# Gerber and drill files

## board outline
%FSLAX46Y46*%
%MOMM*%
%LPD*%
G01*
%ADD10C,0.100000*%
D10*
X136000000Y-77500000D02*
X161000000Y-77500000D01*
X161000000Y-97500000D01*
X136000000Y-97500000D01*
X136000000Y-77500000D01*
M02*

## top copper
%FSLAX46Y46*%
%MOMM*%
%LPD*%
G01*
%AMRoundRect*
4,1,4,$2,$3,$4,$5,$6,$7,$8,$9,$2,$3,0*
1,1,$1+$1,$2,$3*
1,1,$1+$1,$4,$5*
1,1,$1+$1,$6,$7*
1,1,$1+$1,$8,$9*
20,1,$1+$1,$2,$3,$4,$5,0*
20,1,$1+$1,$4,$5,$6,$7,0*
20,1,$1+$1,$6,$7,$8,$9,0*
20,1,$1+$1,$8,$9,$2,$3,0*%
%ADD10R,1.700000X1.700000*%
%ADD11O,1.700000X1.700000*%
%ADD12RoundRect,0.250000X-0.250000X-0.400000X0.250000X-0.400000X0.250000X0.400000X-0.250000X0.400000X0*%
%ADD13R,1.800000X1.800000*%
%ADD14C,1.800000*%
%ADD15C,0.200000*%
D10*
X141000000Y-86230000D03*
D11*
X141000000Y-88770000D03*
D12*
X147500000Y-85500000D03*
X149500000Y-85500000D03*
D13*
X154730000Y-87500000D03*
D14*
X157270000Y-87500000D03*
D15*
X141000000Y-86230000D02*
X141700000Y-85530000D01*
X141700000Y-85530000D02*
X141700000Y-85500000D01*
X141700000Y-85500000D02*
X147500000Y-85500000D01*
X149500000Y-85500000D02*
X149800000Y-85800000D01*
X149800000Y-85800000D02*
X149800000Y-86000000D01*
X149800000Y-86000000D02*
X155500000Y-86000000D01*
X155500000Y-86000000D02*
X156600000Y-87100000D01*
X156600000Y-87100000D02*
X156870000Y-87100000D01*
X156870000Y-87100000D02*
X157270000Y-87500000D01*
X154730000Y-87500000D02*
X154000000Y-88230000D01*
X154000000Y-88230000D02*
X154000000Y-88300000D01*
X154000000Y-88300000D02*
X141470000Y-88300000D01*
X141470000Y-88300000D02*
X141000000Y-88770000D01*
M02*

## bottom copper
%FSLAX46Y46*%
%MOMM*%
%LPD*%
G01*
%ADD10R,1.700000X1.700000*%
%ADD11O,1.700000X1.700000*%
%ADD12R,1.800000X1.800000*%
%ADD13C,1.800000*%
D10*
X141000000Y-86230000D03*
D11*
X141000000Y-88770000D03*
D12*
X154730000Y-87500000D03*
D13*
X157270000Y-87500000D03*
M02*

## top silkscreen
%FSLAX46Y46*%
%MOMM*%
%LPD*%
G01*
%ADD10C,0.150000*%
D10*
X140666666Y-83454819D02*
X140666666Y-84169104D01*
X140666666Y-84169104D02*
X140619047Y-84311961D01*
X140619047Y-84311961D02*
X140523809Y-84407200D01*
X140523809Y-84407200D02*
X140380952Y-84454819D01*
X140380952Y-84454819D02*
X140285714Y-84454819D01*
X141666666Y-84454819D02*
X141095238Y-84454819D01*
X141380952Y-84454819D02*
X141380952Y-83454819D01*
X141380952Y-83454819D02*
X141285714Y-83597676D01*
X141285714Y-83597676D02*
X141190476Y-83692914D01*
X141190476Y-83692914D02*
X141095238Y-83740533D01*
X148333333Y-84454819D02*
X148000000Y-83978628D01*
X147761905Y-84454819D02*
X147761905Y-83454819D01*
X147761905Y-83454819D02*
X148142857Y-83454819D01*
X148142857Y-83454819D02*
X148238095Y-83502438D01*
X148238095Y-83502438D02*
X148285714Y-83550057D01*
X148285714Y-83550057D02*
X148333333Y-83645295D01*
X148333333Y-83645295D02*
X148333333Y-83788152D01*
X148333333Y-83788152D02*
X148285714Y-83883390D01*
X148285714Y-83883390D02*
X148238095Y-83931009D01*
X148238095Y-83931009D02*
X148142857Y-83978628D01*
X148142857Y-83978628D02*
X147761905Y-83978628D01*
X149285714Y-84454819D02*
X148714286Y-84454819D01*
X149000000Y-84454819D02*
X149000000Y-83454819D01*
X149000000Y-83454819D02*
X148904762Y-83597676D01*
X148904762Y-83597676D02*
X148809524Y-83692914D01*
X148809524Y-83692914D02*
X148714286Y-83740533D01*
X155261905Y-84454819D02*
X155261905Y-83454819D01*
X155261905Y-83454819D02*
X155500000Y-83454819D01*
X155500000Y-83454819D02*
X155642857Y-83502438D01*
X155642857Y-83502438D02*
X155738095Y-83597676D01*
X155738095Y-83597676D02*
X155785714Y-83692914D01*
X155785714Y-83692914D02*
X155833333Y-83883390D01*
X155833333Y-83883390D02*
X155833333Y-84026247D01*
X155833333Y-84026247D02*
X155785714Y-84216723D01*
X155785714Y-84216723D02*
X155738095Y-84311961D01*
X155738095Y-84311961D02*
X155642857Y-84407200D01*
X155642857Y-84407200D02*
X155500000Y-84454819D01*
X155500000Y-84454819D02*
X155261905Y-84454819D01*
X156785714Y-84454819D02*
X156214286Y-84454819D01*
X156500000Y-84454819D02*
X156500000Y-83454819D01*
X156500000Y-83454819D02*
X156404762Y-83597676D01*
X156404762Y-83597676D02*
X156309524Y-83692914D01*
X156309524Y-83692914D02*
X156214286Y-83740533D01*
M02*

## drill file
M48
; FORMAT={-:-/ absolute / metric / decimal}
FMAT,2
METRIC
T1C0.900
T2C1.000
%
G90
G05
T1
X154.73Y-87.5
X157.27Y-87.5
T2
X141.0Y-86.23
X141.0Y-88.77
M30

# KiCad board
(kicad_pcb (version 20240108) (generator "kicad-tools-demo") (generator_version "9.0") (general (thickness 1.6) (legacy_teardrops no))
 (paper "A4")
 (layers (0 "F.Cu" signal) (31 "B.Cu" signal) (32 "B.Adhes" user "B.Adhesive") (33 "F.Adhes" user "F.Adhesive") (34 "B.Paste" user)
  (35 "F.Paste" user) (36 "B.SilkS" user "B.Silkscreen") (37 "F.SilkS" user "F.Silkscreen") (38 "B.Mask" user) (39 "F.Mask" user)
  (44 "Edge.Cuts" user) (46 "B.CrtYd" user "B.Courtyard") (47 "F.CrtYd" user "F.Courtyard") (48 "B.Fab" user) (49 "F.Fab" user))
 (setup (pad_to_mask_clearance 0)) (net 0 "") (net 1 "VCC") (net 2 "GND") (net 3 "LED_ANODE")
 (gr_rect (start 136 77.5) (end 161 97.5) (stroke (width 0.1) (type default)) (fill none) (layer "Edge.Cuts"))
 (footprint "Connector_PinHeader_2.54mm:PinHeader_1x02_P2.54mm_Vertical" (layer "F.Cu") (at 141 87.5)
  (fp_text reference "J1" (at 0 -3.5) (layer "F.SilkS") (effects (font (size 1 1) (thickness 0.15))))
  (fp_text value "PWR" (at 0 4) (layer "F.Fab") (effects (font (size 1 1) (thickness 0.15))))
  (pad "1" thru_hole rect (at 0 -1.270) (size 1.7 1.7) (drill 1.0) (layers "*.Cu" "*.Mask") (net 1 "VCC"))
  (pad "2" thru_hole oval (at 0 1.270) (size 1.7 1.7) (drill 1.0) (layers "*.Cu" "*.Mask") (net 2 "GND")))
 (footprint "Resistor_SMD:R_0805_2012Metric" (layer "F.Cu") (at 148.5 85.5 0)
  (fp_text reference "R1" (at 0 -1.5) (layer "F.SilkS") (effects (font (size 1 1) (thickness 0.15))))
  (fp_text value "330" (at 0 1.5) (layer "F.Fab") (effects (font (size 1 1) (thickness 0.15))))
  (pad "1" smd roundrect (at -1.0 0 0) (size 1.0 1.3) (layers "F.Cu" "F.Paste" "F.Mask") (roundrect_rratio 0.25) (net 1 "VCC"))
  (pad "2" smd roundrect (at 1.0 0 0) (size 1.0 1.3) (layers "F.Cu" "F.Paste" "F.Mask") (roundrect_rratio 0.25) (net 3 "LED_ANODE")))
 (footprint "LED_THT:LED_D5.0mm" (layer "F.Cu") (at 156 87.5 0)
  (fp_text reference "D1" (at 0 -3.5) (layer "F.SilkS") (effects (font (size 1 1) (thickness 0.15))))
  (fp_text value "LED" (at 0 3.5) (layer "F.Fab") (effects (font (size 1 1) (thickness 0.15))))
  (pad "1" thru_hole rect (at -1.270 0 0) (size 1.8 1.8) (drill 0.9) (layers "*.Cu" "*.Mask") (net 2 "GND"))
  (pad "2" thru_hole circle (at 1.270 0 0) (size 1.8 1.8) (drill 0.9) (layers "*.Cu" "*.Mask") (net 3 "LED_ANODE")))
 (segment (start 141.0000 86.2300) (end 141.7000 85.5300) (width 0.2) (layer "F.Cu") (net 1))
 (segment (start 141.7000 85.5300) (end 141.7000 85.5000) (width 0.2) (layer "F.Cu") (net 1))
 (segment (start 141.7000 85.5000) (end 147.5000 85.5000) (width 0.2) (layer "F.Cu") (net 1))
 (segment (start 149.5000 85.5000) (end 149.8000 85.8000) (width 0.2) (layer "F.Cu") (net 3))
 (segment (start 149.8000 85.8000) (end 149.8000 86.0000) (width 0.2) (layer "F.Cu") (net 3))
 (segment (start 149.8000 86.0000) (end 155.5000 86.0000) (width 0.2) (layer "F.Cu") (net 3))
 (segment (start 155.5000 86.0000) (end 156.6000 87.1000) (width 0.2) (layer "F.Cu") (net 3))
 (segment (start 156.6000 87.1000) (end 156.8700 87.1000) (width 0.2) (layer "F.Cu") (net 3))
 (segment (start 156.8700 87.1000) (end 157.2700 87.5000) (width 0.2) (layer "F.Cu") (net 3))
 (segment (start 154.7300 87.5000) (end 154.0000 88.2300) (width 0.2) (layer "F.Cu") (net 2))
 (segment (start 154.0000 88.2300) (end 154.0000 88.3000) (width 0.2) (layer "F.Cu") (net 2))
 (segment (start 154.0000 88.3000) (end 141.4700 88.3000) (width 0.2) (layer "F.Cu") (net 2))
 (segment (start 141.4700 88.3000) (end 141.0000 88.7700) (width 0.2) (layer "F.Cu") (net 2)))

